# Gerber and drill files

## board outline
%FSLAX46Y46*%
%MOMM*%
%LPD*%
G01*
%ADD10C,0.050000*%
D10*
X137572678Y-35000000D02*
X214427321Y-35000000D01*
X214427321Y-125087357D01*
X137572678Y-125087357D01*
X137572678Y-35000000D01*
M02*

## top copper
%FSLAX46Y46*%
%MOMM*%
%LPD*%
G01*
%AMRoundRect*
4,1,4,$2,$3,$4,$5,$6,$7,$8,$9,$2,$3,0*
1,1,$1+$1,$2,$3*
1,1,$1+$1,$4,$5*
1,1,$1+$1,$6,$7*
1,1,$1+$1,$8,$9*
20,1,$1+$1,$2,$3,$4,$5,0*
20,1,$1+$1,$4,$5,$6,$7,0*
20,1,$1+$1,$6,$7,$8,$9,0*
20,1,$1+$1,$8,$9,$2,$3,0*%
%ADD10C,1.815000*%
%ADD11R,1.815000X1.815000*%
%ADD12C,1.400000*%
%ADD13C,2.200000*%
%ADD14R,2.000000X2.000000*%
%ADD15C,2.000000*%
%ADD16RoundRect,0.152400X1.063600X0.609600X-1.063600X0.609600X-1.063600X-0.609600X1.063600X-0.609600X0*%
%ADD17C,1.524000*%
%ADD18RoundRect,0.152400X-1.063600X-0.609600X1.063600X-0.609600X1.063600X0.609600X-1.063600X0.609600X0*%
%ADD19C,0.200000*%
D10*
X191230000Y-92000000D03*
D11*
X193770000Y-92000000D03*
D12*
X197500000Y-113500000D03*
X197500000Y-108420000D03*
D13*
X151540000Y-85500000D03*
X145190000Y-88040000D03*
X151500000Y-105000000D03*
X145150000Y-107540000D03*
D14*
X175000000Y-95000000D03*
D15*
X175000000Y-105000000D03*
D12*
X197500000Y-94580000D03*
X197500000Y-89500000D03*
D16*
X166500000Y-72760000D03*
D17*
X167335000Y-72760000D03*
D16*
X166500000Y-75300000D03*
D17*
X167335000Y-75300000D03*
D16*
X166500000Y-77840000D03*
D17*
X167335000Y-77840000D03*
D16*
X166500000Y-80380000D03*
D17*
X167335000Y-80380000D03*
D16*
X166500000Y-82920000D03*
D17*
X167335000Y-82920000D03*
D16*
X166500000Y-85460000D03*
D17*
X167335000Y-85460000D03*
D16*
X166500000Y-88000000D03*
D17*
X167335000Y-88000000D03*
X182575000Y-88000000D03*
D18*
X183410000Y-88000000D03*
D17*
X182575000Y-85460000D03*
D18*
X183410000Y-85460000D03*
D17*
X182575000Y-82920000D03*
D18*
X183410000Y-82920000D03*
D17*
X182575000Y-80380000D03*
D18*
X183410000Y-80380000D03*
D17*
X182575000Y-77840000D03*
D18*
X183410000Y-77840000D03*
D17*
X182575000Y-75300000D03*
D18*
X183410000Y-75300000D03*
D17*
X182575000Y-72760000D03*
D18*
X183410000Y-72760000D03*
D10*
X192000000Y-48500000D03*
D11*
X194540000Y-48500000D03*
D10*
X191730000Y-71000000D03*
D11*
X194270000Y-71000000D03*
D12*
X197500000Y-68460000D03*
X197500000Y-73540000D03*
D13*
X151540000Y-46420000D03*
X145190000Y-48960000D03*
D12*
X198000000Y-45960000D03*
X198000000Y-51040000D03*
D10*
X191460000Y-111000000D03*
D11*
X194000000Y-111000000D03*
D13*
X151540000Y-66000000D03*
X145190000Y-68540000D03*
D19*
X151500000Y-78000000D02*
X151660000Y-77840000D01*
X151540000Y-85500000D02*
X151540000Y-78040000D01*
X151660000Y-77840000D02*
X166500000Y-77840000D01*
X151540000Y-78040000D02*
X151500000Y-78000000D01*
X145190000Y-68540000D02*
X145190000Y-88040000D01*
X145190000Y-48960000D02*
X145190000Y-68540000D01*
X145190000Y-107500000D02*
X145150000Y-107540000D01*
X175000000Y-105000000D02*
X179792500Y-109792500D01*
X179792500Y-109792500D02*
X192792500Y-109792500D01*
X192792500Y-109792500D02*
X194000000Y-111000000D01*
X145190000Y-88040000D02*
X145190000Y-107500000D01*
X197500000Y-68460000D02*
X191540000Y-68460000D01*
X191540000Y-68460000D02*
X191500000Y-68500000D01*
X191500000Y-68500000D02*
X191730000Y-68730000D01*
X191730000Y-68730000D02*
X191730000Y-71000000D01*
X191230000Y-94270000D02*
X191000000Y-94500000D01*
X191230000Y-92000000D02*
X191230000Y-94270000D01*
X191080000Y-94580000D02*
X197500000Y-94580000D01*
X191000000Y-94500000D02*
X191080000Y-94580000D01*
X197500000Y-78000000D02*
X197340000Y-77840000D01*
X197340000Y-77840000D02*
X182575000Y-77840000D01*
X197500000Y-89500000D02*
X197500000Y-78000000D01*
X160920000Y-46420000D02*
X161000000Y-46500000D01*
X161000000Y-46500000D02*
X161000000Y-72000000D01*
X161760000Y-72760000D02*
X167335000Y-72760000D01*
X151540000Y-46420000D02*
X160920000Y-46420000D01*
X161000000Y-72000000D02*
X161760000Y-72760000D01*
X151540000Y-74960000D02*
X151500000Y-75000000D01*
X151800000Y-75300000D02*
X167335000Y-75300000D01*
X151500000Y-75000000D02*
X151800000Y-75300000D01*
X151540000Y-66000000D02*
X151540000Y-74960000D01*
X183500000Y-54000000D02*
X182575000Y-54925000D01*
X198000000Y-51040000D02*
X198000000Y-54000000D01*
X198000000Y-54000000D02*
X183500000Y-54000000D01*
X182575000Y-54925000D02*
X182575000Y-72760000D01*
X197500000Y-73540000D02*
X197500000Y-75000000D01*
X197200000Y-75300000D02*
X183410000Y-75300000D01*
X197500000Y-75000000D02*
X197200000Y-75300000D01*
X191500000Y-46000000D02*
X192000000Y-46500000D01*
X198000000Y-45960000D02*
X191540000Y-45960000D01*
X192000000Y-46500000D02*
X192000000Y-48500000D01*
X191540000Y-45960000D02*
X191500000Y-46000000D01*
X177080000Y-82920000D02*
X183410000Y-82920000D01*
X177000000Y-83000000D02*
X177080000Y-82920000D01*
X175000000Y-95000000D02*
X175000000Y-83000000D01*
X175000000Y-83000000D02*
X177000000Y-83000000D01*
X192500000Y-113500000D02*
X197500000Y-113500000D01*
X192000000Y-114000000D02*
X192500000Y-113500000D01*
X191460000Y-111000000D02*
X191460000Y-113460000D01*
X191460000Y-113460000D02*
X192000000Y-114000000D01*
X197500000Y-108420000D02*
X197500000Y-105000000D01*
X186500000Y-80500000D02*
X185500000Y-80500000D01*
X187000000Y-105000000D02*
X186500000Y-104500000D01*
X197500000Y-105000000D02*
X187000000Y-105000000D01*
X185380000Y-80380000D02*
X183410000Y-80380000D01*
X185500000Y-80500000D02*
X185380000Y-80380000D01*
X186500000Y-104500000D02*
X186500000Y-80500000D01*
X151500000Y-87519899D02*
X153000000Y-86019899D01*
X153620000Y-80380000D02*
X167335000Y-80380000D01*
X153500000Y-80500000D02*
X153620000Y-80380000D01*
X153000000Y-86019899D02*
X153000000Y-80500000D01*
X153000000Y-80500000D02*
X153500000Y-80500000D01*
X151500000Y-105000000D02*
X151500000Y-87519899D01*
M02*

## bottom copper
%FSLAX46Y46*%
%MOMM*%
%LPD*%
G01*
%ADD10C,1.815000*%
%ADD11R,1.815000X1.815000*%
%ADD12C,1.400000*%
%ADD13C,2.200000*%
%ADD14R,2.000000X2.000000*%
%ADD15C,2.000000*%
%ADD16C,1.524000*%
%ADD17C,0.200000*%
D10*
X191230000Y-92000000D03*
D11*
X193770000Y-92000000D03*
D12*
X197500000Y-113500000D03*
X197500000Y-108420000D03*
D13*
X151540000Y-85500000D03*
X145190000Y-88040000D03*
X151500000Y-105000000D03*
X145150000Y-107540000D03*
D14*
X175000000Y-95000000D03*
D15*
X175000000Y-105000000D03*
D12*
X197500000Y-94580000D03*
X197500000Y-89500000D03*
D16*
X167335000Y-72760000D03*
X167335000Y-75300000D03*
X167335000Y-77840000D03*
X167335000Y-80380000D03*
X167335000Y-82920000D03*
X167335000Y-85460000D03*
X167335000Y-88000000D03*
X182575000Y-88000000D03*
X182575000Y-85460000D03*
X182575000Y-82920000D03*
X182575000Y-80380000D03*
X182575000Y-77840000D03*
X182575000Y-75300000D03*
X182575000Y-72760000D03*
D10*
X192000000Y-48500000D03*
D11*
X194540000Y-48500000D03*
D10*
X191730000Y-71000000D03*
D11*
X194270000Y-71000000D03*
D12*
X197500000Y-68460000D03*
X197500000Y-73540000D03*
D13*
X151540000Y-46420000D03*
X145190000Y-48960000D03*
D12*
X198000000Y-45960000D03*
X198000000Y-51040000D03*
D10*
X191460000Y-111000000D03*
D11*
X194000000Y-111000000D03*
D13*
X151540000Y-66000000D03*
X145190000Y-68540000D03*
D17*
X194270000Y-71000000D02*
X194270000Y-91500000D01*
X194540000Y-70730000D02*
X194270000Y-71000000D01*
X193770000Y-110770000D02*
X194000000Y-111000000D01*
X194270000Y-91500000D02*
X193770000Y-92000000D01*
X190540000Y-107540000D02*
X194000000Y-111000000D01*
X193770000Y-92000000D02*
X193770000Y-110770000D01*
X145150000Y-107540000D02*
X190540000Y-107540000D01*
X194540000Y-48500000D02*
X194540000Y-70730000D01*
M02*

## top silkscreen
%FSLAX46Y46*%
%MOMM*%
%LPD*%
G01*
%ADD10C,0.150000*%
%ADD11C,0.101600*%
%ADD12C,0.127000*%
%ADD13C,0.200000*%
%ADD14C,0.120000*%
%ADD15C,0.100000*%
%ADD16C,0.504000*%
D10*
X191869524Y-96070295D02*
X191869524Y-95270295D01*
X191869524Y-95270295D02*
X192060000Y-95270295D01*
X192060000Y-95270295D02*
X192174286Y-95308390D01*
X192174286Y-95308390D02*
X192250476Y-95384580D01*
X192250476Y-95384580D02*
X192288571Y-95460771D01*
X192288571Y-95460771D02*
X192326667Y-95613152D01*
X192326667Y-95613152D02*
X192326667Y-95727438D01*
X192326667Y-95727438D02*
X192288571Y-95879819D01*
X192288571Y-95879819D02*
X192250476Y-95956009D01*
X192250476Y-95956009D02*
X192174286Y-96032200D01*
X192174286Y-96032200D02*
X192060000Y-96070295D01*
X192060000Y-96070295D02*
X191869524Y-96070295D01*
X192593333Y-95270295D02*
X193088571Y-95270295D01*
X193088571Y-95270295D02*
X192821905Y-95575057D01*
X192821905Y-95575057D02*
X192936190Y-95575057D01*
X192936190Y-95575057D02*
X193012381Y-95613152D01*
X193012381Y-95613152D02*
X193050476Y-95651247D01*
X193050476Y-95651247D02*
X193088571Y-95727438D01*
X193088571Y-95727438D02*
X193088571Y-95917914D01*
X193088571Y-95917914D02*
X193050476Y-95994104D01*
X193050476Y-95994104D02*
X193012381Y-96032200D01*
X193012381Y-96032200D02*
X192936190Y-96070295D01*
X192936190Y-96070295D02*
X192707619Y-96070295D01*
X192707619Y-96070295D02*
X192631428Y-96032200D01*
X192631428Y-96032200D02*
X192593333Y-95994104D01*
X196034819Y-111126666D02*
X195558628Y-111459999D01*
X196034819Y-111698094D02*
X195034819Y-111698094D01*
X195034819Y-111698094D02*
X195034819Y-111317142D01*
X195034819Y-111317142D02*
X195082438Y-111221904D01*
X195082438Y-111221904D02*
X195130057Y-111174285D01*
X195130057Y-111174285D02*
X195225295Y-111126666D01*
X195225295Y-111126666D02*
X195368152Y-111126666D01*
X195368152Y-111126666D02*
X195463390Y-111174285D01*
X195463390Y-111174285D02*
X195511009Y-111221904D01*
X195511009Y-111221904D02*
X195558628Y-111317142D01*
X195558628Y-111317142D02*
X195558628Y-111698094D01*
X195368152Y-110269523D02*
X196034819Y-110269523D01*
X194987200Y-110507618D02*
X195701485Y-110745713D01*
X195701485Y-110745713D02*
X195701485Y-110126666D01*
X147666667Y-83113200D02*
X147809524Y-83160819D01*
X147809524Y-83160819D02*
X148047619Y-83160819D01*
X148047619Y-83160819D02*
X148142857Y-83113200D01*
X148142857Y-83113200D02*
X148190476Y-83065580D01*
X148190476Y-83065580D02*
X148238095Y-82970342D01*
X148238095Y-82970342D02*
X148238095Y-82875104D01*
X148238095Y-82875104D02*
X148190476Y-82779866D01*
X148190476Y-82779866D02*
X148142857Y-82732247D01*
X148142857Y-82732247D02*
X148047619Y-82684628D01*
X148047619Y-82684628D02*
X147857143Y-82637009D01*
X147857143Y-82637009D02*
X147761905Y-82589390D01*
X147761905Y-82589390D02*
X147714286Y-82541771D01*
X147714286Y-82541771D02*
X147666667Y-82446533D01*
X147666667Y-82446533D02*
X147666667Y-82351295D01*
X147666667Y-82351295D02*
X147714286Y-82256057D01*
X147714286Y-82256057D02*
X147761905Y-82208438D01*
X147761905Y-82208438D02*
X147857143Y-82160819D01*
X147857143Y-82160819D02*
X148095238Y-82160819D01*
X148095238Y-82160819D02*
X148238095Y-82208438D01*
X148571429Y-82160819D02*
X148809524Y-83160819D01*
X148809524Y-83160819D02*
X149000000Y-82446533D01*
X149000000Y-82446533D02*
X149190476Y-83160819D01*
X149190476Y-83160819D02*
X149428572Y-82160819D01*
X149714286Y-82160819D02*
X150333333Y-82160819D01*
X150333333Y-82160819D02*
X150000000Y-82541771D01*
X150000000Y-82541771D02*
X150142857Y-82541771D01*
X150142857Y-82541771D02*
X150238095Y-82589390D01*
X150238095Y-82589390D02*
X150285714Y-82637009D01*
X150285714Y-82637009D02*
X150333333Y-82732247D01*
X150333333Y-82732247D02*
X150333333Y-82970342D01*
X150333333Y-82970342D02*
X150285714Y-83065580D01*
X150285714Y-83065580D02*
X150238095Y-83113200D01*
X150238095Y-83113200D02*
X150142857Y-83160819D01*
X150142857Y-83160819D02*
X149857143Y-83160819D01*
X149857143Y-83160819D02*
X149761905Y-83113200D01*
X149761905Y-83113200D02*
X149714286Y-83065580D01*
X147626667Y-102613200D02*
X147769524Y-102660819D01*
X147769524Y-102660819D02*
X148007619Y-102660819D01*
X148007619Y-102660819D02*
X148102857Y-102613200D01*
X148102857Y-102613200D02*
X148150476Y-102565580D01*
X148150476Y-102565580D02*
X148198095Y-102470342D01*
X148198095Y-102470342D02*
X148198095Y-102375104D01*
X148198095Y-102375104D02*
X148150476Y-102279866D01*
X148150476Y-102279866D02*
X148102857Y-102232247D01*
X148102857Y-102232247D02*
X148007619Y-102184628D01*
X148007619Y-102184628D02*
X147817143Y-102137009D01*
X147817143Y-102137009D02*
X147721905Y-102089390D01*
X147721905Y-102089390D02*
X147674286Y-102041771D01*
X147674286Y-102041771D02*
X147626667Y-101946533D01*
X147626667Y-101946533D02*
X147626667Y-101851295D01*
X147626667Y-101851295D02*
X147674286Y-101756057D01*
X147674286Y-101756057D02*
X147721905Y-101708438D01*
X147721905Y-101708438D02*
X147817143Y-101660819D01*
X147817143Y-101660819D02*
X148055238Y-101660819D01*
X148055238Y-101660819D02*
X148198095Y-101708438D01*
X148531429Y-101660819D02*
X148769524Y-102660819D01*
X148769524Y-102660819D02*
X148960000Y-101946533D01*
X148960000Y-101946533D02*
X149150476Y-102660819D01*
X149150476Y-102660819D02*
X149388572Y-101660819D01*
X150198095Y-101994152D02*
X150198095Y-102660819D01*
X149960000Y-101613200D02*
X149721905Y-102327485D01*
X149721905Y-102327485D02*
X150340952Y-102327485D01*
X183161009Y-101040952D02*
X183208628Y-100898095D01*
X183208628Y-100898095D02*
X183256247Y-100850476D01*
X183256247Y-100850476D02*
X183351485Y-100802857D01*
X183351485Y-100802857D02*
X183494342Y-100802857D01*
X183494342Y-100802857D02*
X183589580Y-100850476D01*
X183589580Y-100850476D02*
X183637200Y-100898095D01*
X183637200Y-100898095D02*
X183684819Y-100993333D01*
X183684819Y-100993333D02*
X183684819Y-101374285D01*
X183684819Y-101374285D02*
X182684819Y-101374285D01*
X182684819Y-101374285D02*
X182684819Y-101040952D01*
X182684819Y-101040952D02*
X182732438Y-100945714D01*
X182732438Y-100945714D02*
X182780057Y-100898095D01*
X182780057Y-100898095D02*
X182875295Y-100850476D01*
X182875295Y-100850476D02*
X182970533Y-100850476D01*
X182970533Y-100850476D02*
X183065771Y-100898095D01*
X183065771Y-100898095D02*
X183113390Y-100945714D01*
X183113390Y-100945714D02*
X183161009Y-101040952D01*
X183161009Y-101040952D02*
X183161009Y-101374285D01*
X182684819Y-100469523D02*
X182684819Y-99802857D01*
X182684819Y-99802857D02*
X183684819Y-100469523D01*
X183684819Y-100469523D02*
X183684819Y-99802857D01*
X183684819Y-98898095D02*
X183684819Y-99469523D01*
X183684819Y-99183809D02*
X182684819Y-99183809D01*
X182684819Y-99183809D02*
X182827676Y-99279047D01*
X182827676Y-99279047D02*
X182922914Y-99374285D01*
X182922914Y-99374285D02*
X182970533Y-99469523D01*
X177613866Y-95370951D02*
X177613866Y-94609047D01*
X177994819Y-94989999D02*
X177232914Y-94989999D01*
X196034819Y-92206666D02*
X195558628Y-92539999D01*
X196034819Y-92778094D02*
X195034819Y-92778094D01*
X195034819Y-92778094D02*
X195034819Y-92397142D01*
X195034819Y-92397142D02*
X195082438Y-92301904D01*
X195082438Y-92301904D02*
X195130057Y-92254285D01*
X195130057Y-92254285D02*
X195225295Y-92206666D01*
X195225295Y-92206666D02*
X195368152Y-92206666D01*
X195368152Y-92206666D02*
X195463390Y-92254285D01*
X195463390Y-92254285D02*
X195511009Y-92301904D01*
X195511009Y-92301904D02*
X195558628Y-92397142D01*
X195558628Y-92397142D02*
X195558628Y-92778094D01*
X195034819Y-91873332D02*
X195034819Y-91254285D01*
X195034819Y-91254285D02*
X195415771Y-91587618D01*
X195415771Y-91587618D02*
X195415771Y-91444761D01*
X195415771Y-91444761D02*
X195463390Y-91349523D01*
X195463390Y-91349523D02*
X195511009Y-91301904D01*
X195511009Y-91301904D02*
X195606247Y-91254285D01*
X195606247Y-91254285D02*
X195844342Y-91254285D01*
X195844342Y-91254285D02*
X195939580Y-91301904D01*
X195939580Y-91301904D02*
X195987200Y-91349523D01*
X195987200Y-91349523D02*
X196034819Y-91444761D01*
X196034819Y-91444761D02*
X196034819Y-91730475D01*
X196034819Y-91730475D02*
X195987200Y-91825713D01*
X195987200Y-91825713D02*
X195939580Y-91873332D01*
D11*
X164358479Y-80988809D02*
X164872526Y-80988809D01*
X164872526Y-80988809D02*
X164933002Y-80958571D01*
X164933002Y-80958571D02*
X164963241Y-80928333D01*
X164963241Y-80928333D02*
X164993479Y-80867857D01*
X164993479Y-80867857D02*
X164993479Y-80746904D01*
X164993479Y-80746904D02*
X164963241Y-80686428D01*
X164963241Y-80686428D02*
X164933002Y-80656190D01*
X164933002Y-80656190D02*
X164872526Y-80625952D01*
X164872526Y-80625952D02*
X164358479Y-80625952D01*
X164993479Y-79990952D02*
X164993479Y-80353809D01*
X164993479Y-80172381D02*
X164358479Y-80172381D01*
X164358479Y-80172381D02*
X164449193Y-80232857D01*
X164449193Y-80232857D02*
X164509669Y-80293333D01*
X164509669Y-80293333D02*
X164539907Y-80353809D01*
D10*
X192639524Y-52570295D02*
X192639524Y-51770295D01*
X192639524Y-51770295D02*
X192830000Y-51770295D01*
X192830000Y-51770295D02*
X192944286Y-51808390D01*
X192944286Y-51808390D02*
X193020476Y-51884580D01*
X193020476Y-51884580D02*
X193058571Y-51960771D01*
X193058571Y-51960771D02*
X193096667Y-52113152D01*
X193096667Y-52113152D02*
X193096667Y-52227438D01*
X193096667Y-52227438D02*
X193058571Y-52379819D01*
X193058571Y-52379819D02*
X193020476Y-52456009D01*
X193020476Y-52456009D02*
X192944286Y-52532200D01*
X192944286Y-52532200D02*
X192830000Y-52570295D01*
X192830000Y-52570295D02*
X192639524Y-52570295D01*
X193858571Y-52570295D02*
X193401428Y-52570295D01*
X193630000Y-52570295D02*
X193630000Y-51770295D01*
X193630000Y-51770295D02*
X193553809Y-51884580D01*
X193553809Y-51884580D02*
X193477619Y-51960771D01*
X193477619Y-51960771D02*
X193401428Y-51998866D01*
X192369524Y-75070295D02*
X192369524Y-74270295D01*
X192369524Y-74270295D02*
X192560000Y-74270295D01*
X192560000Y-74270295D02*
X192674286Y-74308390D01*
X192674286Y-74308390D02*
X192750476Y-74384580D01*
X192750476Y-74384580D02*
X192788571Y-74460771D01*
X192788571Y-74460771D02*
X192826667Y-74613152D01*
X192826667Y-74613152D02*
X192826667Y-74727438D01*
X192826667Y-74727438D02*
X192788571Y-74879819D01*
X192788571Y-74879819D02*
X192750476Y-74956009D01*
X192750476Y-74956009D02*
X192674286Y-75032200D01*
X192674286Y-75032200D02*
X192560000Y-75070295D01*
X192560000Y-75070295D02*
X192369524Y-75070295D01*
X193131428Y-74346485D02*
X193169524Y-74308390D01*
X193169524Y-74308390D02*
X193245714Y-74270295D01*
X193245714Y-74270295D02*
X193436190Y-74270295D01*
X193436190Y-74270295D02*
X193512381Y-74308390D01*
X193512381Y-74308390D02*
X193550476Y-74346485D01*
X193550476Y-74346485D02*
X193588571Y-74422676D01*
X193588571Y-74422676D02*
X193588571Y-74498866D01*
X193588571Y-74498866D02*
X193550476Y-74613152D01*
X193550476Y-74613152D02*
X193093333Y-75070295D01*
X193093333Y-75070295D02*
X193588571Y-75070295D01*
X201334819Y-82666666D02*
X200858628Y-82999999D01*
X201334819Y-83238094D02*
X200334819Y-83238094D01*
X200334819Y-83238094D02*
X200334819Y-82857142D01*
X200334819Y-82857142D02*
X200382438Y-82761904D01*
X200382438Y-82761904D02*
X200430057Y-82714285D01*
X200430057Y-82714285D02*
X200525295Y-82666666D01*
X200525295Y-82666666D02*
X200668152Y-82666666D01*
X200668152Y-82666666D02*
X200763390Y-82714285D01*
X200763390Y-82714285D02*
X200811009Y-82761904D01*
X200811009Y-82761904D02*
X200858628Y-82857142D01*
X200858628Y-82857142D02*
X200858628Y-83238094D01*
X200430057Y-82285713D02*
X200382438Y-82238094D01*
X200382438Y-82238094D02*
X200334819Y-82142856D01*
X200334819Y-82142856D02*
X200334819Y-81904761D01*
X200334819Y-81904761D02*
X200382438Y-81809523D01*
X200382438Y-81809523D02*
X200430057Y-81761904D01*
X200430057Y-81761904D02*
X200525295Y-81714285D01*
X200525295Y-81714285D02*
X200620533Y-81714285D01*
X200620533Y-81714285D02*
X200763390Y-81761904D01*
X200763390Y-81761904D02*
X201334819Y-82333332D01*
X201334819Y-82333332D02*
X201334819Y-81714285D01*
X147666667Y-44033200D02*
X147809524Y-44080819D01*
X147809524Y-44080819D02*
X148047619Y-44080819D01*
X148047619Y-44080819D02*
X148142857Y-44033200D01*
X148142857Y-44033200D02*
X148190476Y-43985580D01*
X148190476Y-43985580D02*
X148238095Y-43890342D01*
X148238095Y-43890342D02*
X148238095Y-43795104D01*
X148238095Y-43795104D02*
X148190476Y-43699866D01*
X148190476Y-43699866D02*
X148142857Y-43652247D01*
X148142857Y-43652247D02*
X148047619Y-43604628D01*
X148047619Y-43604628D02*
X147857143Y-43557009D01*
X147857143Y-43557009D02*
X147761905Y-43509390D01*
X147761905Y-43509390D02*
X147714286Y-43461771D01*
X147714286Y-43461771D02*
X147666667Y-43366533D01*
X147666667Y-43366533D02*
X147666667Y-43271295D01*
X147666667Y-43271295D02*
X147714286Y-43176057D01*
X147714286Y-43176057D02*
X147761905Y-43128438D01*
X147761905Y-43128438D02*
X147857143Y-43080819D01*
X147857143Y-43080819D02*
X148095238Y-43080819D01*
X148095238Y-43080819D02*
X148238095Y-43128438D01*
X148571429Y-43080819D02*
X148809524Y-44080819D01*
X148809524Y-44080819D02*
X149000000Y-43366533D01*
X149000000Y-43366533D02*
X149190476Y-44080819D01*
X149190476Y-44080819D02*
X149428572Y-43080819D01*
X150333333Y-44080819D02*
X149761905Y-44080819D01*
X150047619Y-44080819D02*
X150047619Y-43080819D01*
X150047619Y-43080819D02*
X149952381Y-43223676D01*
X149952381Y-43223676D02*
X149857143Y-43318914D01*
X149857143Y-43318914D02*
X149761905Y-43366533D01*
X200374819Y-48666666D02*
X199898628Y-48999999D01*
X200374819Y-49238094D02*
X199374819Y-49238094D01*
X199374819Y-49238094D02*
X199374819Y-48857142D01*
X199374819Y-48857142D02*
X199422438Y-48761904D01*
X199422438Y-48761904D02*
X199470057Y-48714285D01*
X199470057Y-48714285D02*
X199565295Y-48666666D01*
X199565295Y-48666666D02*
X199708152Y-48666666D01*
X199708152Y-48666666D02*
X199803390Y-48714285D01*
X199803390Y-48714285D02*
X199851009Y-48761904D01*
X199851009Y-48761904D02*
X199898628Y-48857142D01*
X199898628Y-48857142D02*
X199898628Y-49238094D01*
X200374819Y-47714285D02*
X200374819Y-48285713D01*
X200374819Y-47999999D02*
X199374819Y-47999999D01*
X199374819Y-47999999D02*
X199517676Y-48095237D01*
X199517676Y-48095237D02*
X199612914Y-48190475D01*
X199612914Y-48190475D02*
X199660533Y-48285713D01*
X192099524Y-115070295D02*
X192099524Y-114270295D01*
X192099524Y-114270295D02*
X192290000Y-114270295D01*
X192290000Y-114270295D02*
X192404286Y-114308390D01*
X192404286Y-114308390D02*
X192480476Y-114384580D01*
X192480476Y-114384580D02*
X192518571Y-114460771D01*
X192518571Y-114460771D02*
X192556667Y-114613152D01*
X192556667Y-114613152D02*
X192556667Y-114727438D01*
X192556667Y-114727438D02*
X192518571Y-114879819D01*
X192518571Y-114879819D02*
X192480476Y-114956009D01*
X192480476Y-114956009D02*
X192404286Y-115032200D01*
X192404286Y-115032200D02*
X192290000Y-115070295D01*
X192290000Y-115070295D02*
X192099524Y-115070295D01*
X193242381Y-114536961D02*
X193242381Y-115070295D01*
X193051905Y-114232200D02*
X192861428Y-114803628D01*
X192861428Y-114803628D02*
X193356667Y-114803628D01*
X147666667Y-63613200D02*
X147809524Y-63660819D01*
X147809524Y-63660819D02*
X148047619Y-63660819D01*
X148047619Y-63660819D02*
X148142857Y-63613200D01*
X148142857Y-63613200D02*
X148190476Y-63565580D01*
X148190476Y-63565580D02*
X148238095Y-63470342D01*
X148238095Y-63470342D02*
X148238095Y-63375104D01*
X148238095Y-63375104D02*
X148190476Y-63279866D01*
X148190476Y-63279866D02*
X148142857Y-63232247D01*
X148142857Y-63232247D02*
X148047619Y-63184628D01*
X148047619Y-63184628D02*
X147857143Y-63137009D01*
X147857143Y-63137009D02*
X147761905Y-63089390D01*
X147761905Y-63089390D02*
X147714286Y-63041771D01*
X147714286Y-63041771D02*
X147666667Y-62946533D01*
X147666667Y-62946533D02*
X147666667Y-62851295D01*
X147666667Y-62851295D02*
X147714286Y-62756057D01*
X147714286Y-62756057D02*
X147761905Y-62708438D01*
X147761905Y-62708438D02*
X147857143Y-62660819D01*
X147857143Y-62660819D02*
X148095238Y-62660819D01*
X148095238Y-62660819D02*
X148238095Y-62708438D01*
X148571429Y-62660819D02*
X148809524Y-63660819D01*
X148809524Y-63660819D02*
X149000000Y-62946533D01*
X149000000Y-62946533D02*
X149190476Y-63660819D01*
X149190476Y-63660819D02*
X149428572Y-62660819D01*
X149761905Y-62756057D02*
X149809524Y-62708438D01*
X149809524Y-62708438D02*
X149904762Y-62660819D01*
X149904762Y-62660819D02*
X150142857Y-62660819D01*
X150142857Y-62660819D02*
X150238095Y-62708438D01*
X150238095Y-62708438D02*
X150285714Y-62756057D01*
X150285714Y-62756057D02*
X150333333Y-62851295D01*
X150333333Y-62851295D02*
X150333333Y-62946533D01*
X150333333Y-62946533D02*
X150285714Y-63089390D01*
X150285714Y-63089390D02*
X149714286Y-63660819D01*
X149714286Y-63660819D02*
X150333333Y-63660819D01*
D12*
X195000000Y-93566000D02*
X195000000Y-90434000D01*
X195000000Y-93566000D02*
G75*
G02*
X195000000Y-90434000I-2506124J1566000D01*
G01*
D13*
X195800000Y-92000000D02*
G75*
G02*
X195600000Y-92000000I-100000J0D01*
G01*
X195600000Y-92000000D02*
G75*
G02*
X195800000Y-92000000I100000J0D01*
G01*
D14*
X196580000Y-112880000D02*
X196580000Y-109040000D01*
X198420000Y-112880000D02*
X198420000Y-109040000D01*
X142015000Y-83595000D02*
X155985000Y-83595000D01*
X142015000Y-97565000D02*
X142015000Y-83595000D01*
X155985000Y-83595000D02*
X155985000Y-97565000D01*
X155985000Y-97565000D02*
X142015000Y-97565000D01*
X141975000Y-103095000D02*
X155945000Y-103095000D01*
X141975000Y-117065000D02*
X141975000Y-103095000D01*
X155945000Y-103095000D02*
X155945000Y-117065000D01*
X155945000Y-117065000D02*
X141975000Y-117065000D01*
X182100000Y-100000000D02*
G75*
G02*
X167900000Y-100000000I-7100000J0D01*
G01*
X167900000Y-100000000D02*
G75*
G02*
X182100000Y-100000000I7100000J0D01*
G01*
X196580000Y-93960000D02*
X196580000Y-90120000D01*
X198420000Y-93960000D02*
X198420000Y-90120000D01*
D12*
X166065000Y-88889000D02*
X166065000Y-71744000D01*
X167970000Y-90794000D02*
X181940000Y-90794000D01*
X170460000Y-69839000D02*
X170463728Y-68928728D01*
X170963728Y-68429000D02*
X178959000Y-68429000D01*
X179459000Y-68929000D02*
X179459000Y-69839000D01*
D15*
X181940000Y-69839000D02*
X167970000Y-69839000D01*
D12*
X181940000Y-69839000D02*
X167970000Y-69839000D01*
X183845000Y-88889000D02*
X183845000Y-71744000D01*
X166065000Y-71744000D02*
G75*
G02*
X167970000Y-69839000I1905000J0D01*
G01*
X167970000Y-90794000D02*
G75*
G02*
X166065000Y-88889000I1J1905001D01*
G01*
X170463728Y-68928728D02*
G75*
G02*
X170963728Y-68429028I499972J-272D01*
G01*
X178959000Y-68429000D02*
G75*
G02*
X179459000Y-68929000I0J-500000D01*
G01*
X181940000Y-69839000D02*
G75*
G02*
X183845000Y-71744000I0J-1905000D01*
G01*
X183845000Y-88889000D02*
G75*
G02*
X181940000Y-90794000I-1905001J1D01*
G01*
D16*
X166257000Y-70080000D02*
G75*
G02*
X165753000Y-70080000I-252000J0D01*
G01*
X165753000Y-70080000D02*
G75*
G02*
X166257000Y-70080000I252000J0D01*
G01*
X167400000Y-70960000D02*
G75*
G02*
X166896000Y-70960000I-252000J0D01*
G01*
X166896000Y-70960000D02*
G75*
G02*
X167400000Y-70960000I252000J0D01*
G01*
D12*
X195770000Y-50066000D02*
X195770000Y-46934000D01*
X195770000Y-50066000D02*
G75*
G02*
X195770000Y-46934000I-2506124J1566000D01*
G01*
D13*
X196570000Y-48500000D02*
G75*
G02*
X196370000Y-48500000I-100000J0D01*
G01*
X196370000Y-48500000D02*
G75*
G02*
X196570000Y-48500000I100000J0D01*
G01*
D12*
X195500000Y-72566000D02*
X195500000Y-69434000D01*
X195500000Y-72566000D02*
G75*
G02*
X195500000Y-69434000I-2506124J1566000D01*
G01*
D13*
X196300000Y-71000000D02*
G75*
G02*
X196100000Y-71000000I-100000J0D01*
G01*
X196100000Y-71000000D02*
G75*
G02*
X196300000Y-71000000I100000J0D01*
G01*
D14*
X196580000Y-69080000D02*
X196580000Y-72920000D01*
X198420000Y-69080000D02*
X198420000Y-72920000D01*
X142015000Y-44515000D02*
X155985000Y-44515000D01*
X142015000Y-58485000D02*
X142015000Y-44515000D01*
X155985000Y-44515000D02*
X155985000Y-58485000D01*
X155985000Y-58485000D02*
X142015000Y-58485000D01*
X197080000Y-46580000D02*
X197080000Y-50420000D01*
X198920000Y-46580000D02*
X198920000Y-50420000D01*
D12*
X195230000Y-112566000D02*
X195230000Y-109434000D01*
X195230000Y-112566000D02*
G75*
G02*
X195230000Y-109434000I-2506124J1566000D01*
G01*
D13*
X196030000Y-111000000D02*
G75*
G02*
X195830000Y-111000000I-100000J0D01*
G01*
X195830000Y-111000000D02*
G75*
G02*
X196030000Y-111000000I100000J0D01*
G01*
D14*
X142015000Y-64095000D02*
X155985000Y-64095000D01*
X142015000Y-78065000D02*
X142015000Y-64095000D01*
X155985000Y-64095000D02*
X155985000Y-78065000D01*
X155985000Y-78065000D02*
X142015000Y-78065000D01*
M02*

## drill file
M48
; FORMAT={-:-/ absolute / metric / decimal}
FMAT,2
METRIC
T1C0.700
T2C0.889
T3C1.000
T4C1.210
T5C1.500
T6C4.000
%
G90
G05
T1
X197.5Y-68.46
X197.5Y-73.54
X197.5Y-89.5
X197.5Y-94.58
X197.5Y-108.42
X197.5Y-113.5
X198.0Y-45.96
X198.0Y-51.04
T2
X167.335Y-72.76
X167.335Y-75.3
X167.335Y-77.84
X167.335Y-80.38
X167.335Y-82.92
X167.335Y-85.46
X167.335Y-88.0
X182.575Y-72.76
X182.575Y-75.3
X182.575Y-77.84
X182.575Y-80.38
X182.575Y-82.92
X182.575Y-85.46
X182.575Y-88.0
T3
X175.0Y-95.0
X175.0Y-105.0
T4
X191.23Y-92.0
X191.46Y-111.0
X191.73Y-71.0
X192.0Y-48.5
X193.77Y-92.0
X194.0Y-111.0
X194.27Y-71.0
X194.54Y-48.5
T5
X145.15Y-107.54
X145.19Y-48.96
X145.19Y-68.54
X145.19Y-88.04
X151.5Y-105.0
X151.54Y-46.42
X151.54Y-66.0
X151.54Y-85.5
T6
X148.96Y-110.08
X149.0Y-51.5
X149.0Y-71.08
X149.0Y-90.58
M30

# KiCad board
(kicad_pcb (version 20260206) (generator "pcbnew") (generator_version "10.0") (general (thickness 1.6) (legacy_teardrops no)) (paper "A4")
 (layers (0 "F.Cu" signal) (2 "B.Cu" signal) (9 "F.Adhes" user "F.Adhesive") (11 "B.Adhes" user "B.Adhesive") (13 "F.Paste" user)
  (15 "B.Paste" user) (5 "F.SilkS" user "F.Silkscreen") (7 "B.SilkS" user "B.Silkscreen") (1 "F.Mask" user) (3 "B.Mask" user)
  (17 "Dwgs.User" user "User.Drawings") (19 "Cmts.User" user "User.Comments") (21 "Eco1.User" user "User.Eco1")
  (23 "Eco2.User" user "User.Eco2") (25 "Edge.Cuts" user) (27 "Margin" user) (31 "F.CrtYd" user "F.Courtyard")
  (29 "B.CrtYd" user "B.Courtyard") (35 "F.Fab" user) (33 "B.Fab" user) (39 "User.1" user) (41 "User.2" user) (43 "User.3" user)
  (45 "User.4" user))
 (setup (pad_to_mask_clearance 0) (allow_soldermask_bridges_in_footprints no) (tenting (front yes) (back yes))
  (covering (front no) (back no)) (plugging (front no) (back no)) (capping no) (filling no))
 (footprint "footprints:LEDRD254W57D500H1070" (layer "F.Cu") (at 192.5 92 180)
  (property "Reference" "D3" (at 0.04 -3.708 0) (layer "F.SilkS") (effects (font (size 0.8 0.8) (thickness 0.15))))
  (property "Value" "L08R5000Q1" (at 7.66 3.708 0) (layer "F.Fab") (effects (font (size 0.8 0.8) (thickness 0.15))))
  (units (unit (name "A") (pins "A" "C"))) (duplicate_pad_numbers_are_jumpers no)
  (fp_line (start -2.5 -1.566) (end -2.5 1.566) (stroke (width 0.127) (type solid)) (layer "F.SilkS"))
  (fp_arc (start -2.5 -1.566) (mid 2.961291 0) (end -2.5 1.566) (stroke (width 0.127) (type solid)) (layer "F.SilkS"))
  (fp_circle (center -3.2 0) (end -3.1 0) (stroke (width 0.2) (type solid)) (fill no) (layer "F.SilkS"))
  (pad "A" thru_hole circle (at 1.27 0 180) (size 1.815 1.815) (drill 1.21) (layers "*.Cu" "*.Mask") (remove_unused_layers no)
   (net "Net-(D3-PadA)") (solder_mask_margin 0.102))
  (pad "C" thru_hole rect (at -1.27 0 180) (size 1.815 1.815) (drill 1.21) (layers "*.Cu" "*.Mask") (remove_unused_layers no) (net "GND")
   (solder_mask_margin 0.102)))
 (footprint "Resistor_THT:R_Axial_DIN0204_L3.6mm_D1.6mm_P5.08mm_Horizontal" (layer "F.Cu") (at 197.5 113.5 90)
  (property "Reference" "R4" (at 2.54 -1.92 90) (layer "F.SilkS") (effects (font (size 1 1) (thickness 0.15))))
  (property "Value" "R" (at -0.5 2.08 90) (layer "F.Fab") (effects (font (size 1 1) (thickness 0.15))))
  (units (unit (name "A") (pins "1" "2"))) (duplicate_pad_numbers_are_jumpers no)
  (fp_line (start 0.62 -0.92) (end 4.46 -0.92) (stroke (width 0.12) (type solid)) (layer "F.SilkS"))
  (fp_line (start 0.62 0.92) (end 4.46 0.92) (stroke (width 0.12) (type solid)) (layer "F.SilkS"))
  (pad "1" thru_hole circle (at 0 0 90) (size 1.4 1.4) (drill 0.7) (layers "*.Cu" "*.Mask") (remove_unused_layers no) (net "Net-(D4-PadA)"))
  (pad "2" thru_hole circle (at 5.08 0 90) (size 1.4 1.4) (drill 0.7) (layers "*.Cu" "*.Mask") (remove_unused_layers no) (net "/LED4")))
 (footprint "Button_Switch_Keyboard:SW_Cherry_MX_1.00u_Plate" (layer "F.Cu") (at 151.54 85.5)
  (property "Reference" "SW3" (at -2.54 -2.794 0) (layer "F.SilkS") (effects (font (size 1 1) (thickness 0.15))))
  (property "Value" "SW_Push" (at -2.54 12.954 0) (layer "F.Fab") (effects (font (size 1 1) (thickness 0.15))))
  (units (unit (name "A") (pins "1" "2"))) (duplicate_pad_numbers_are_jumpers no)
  (fp_line (start -9.525 -1.905) (end 4.445 -1.905) (stroke (width 0.12) (type solid)) (layer "F.SilkS"))
  (fp_line (start -9.525 12.065) (end -9.525 -1.905) (stroke (width 0.12) (type solid)) (layer "F.SilkS"))
  (fp_line (start 4.445 -1.905) (end 4.445 12.065) (stroke (width 0.12) (type solid)) (layer "F.SilkS"))
  (fp_line (start 4.445 12.065) (end -9.525 12.065) (stroke (width 0.12) (type solid)) (layer "F.SilkS"))
  (pad "" np_thru_hole circle (at -2.54 5.08) (size 4 4) (drill 4) (layers "*.Cu" "*.Mask"))
  (pad "1" thru_hole circle (at 0 0) (size 2.2 2.2) (drill 1.5) (layers "*.Cu" "*.Mask") (remove_unused_layers no) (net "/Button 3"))
  (pad "2" thru_hole circle (at -6.35 2.54) (size 2.2 2.2) (drill 1.5) (layers "*.Cu" "*.Mask") (remove_unused_layers no) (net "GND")))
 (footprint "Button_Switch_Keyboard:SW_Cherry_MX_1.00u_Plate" (layer "F.Cu") (at 151.5 105)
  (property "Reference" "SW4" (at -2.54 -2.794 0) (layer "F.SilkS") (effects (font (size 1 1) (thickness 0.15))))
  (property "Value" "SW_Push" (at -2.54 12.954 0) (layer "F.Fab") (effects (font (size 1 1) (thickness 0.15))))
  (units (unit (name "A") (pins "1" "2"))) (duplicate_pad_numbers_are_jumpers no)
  (fp_line (start -9.525 -1.905) (end 4.445 -1.905) (stroke (width 0.12) (type solid)) (layer "F.SilkS"))
  (fp_line (start -9.525 12.065) (end -9.525 -1.905) (stroke (width 0.12) (type solid)) (layer "F.SilkS"))
  (fp_line (start 4.445 -1.905) (end 4.445 12.065) (stroke (width 0.12) (type solid)) (layer "F.SilkS"))
  (fp_line (start 4.445 12.065) (end -9.525 12.065) (stroke (width 0.12) (type solid)) (layer "F.SilkS"))
  (pad "" np_thru_hole circle (at -2.54 5.08) (size 4 4) (drill 4) (layers "*.Cu" "*.Mask"))
  (pad "1" thru_hole circle (at 0 0) (size 2.2 2.2) (drill 1.5) (layers "*.Cu" "*.Mask") (remove_unused_layers no) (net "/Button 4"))
  (pad "2" thru_hole circle (at -6.35 2.54) (size 2.2 2.2) (drill 1.5) (layers "*.Cu" "*.Mask") (remove_unused_layers no) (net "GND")))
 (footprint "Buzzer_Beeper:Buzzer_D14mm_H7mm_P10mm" (layer "F.Cu") (at 175 95 -90)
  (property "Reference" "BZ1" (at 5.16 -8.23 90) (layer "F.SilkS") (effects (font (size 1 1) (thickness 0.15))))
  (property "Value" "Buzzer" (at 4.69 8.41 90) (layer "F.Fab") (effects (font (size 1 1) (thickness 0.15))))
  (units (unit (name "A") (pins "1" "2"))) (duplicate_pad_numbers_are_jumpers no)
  (fp_circle (center 5 0) (end 12.1 0) (stroke (width 0.12) (type solid)) (fill no) (layer "F.SilkS"))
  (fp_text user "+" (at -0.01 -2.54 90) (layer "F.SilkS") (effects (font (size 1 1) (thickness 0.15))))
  (pad "1" thru_hole rect (at 0 0 270) (size 2 2) (drill 1) (layers "*.Cu" "*.Mask") (remove_unused_layers no) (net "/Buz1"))
  (pad "2" thru_hole circle (at 10 0 270) (size 2 2) (drill 1) (layers "*.Cu" "*.Mask") (remove_unused_layers no) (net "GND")))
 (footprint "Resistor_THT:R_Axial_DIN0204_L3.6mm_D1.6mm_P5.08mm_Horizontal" (layer "F.Cu") (at 197.5 94.58 90)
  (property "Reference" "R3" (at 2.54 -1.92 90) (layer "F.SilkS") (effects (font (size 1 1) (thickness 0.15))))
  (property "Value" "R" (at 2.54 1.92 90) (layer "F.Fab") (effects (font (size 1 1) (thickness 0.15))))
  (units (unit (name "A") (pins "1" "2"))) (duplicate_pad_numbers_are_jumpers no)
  (fp_line (start 0.62 -0.92) (end 4.46 -0.92) (stroke (width 0.12) (type solid)) (layer "F.SilkS"))
  (fp_line (start 0.62 0.92) (end 4.46 0.92) (stroke (width 0.12) (type solid)) (layer "F.SilkS"))
  (pad "1" thru_hole circle (at 0 0 90) (size 1.4 1.4) (drill 0.7) (layers "*.Cu" "*.Mask") (remove_unused_layers no) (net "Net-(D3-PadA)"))
  (pad "2" thru_hole circle (at 5.08 0 90) (size 1.4 1.4) (drill 0.7) (layers "*.Cu" "*.Mask") (remove_unused_layers no) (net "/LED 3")))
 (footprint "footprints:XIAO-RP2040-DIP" (layer "F.Cu") (at 174.955 80.38 90)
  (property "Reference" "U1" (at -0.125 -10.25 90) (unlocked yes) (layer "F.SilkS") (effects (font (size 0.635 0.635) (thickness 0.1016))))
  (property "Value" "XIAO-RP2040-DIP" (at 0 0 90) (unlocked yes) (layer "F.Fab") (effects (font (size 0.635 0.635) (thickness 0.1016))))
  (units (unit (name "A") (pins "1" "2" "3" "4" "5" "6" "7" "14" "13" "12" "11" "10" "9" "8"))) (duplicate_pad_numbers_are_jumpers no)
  (fp_line (start -8.509 -8.89) (end 8.636 -8.89) (stroke (width 0.127) (type solid)) (layer "F.SilkS"))
  (fp_line (start -10.414 -6.985) (end -10.414 6.985) (stroke (width 0.127) (type solid)) (layer "F.SilkS"))
  (fp_line (start 10.541 -4.495) (end 11.451272 -4.491272) (stroke (width 0.127) (type solid)) (layer "F.SilkS"))
  (fp_line (start 11.951 -3.991272) (end 11.951 4.004) (stroke (width 0.127) (type solid)) (layer "F.SilkS"))
  (fp_line (start 11.451 4.504) (end 10.541 4.504) (stroke (width 0.127) (type solid)) (layer "F.SilkS"))
  (fp_line (start 10.541 6.985) (end 10.541 -6.985) (stroke (width 0.1) (type solid)) (layer "F.SilkS"))
  (fp_line (start 10.541 6.985) (end 10.541 -6.985) (stroke (width 0.127) (type solid)) (layer "F.SilkS"))
  (fp_line (start -8.509 8.89) (end 8.636 8.89) (stroke (width 0.127) (type solid)) (layer "F.SilkS"))
  (fp_arc (start 8.636 -8.89) (mid 9.983038 -8.332038) (end 10.541 -6.985) (stroke (width 0.127) (type solid)) (layer "F.SilkS"))
  (fp_arc (start -10.414 -6.985) (mid -9.856038 -8.332038) (end -8.509 -8.89) (stroke (width 0.127) (type solid)) (layer "F.SilkS"))
  (fp_arc (start 11.451272 -4.491272) (mid 11.804644 -4.344724) (end 11.951 -3.991272) (stroke (width 0.127) (type default))
   (layer "F.SilkS"))
  (fp_arc (start 11.951 4.004) (mid 11.804553 4.357553) (end 11.451 4.504) (stroke (width 0.127) (type default)) (layer "F.SilkS"))
  (fp_arc (start 10.541 6.985) (mid 9.983038 8.332038) (end 8.636 8.89) (stroke (width 0.127) (type solid)) (layer "F.SilkS"))
  (fp_arc (start -8.509 8.89) (mid -9.856038 8.332038) (end -10.414 6.985) (stroke (width 0.127) (type solid)) (layer "F.SilkS"))
  (fp_circle (center 10.3 -8.95) (end 10.554 -8.95) (stroke (width 0.5) (type solid)) (fill yes) (layer "F.SilkS"))
  (fp_circle (center 9.42 -7.807) (end 9.674 -7.807) (stroke (width 0.5) (type solid)) (fill yes) (layer "F.SilkS"))
  (pad "1" smd roundrect (at 7.62 -8.455 180) (size 2.432 1.524) (layers "F.Cu" "F.Mask") (roundrect_rratio 0.1) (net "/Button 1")
   (thermal_bridge_angle 45))
  (pad "1" thru_hole circle (at 7.62 -7.62 180) (size 1.524 1.524) (drill 0.889) (layers "*.Cu" "*.Mask") (remove_unused_layers no)
   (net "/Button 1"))
  (pad "2" smd roundrect (at 5.08 -8.455 180) (size 2.432 1.524) (layers "F.Cu" "F.Mask") (roundrect_rratio 0.1) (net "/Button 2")
   (thermal_bridge_angle 45))
  (pad "2" thru_hole circle (at 5.08 -7.62 180) (size 1.524 1.524) (drill 0.889) (layers "*.Cu" "*.Mask") (remove_unused_layers no)
   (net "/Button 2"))
  (pad "3" smd roundrect (at 2.54 -8.455 180) (size 2.432 1.524) (layers "F.Cu" "F.Mask") (roundrect_rratio 0.1) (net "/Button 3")
   (thermal_bridge_angle 45))
  (pad "3" thru_hole circle (at 2.54 -7.62 180) (size 1.524 1.524) (drill 0.889) (layers "*.Cu" "*.Mask") (remove_unused_layers no)
   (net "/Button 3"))
  (pad "4" smd roundrect (at 0 -8.455 180) (size 2.432 1.524) (layers "F.Cu" "F.Mask") (roundrect_rratio 0.1) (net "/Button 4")
   (thermal_bridge_angle 45))
  (pad "4" thru_hole circle (at 0 -7.62 180) (size 1.524 1.524) (drill 0.889) (layers "*.Cu" "*.Mask") (remove_unused_layers no)
   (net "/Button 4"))
  (pad "5" smd roundrect (at -2.54 -8.455 180) (size 2.432 1.524) (layers "F.Cu" "F.Mask") (roundrect_rratio 0.1)
   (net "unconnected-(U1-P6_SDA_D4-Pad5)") (thermal_bridge_angle 45))
  (pad "5" thru_hole circle (at -2.54 -7.62 180) (size 1.524 1.524) (drill 0.889) (layers "*.Cu" "*.Mask") (remove_unused_layers no)
   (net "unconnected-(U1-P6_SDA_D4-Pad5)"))
  (pad "6" smd roundrect (at -5.08 -8.455 180) (size 2.432 1.524) (layers "F.Cu" "F.Mask") (roundrect_rratio 0.1)
   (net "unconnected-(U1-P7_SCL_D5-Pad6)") (thermal_bridge_angle 45))
  (pad "6" thru_hole circle (at -5.08 -7.62 180) (size 1.524 1.524) (drill 0.889) (layers "*.Cu" "*.Mask") (remove_unused_layers no)
   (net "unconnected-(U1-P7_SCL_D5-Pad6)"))
  (pad "7" smd roundrect (at -7.62 -8.455 180) (size 2.432 1.524) (layers "F.Cu" "F.Mask") (roundrect_rratio 0.1)
   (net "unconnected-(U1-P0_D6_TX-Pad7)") (thermal_bridge_angle 45))
  (pad "7" thru_hole circle (at -7.62 -7.62 180) (size 1.524 1.524) (drill 0.889) (layers "*.Cu" "*.Mask") (remove_unused_layers no)
   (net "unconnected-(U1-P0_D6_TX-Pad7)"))
  (pad "8" thru_hole circle (at -7.62 7.62) (size 1.524 1.524) (drill 0.889) (layers "*.Cu" "*.Mask") (remove_unused_layers no)
   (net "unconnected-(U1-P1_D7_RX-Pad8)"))
  (pad "8" smd roundrect (at -7.62 8.455) (size 2.432 1.524) (layers "F.Cu" "F.Mask") (roundrect_rratio 0.1)
   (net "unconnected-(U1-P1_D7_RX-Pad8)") (thermal_bridge_angle 45))
  (pad "9" thru_hole circle (at -5.08 7.62) (size 1.524 1.524) (drill 0.889) (layers "*.Cu" "*.Mask") (remove_unused_layers no)
   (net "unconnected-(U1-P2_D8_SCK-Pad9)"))
  (pad "9" smd roundrect (at -5.08 8.455) (size 2.432 1.524) (layers "F.Cu" "F.Mask") (roundrect_rratio 0.1)
   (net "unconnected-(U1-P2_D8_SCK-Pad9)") (thermal_bridge_angle 45))
  (pad "10" thru_hole circle (at -2.54 7.62) (size 1.524 1.524) (drill 0.889) (layers "*.Cu" "*.Mask") (remove_unused_layers no)
   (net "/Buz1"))
  (pad "10" smd roundrect (at -2.54 8.455) (size 2.432 1.524) (layers "F.Cu" "F.Mask") (roundrect_rratio 0.1) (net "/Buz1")
   (thermal_bridge_angle 45))
  (pad "11" thru_hole circle (at 0 7.62) (size 1.524 1.524) (drill 0.889) (layers "*.Cu" "*.Mask") (remove_unused_layers no) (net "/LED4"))
  (pad "11" smd roundrect (at 0 8.455) (size 2.432 1.524) (layers "F.Cu" "F.Mask") (roundrect_rratio 0.1) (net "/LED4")
   (thermal_bridge_angle 45))
  (pad "12" thru_hole circle (at 2.54 7.62) (size 1.524 1.524) (drill 0.889) (layers "*.Cu" "*.Mask") (remove_unused_layers no)
   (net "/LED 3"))
  (pad "12" smd roundrect (at 2.54 8.455) (size 2.432 1.524) (layers "F.Cu" "F.Mask") (roundrect_rratio 0.1) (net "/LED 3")
   (thermal_bridge_angle 45))
  (pad "13" thru_hole circle (at 5.08 7.62) (size 1.524 1.524) (drill 0.889) (layers "*.Cu" "*.Mask") (remove_unused_layers no)
   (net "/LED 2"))
  (pad "13" smd roundrect (at 5.08 8.455) (size 2.432 1.524) (layers "F.Cu" "F.Mask") (roundrect_rratio 0.1) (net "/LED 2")
   (thermal_bridge_angle 45))
  (pad "14" thru_hole circle (at 7.62 7.62) (size 1.524 1.524) (drill 0.889) (layers "*.Cu" "*.Mask") (remove_unused_layers no)
   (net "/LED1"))
  (pad "14" smd roundrect (at 7.62 8.455) (size 2.432 1.524) (layers "F.Cu" "F.Mask") (roundrect_rratio 0.1) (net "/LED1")
   (thermal_bridge_angle 45)))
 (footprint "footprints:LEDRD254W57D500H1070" (layer "F.Cu") (at 193.27 48.5 180)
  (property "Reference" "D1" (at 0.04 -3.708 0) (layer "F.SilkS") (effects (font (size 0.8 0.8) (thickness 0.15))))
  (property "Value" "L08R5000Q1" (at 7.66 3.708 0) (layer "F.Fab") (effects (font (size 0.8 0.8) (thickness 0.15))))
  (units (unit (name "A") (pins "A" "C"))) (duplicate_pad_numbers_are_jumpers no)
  (fp_line (start -2.5 -1.566) (end -2.5 1.566) (stroke (width 0.127) (type solid)) (layer "F.SilkS"))
  (fp_arc (start -2.5 -1.566) (mid 2.961291 0) (end -2.5 1.566) (stroke (width 0.127) (type solid)) (layer "F.SilkS"))
  (fp_circle (center -3.2 0) (end -3.1 0) (stroke (width 0.2) (type solid)) (fill no) (layer "F.SilkS"))
  (pad "A" thru_hole circle (at 1.27 0 180) (size 1.815 1.815) (drill 1.21) (layers "*.Cu" "*.Mask") (remove_unused_layers no)
   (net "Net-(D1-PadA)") (solder_mask_margin 0.102))
  (pad "C" thru_hole rect (at -1.27 0 180) (size 1.815 1.815) (drill 1.21) (layers "*.Cu" "*.Mask") (remove_unused_layers no) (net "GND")
   (solder_mask_margin 0.102)))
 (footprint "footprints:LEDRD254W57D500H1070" (layer "F.Cu") (at 193 71 180)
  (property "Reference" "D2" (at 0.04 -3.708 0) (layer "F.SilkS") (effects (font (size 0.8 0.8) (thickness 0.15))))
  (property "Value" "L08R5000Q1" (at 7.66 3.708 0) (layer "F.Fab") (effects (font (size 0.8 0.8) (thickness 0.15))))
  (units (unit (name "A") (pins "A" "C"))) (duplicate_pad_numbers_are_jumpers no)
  (fp_line (start -2.5 -1.566) (end -2.5 1.566) (stroke (width 0.127) (type solid)) (layer "F.SilkS"))
  (fp_arc (start -2.5 -1.566) (mid 2.961291 0) (end -2.5 1.566) (stroke (width 0.127) (type solid)) (layer "F.SilkS"))
  (fp_circle (center -3.2 0) (end -3.1 0) (stroke (width 0.2) (type solid)) (fill no) (layer "F.SilkS"))
  (pad "A" thru_hole circle (at 1.27 0 180) (size 1.815 1.815) (drill 1.21) (layers "*.Cu" "*.Mask") (remove_unused_layers no)
   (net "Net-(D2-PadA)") (solder_mask_margin 0.102))
  (pad "C" thru_hole rect (at -1.27 0 180) (size 1.815 1.815) (drill 1.21) (layers "*.Cu" "*.Mask") (remove_unused_layers no) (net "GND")
   (solder_mask_margin 0.102)))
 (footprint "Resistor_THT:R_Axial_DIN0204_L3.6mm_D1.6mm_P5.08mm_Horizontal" (layer "F.Cu") (at 197.5 68.46 -90)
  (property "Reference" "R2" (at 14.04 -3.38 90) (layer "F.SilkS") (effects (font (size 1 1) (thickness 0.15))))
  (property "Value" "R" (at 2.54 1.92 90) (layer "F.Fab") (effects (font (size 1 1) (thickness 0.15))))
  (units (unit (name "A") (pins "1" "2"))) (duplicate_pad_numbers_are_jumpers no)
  (fp_line (start 0.62 0.92) (end 4.46 0.92) (stroke (width 0.12) (type solid)) (layer "F.SilkS"))
  (fp_line (start 0.62 -0.92) (end 4.46 -0.92) (stroke (width 0.12) (type solid)) (layer "F.SilkS"))
  (pad "1" thru_hole circle (at 0 0 270) (size 1.4 1.4) (drill 0.7) (layers "*.Cu" "*.Mask") (remove_unused_layers no) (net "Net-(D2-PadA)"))
  (pad "2" thru_hole circle (at 5.08 0 270) (size 1.4 1.4) (drill 0.7) (layers "*.Cu" "*.Mask") (remove_unused_layers no) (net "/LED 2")))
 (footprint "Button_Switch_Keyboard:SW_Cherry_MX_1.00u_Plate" (layer "F.Cu") (at 151.54 46.42)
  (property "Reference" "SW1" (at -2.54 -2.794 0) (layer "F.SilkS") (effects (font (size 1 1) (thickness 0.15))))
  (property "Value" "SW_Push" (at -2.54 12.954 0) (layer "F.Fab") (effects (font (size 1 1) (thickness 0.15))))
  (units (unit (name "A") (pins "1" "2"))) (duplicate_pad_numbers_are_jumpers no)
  (fp_line (start -9.525 -1.905) (end 4.445 -1.905) (stroke (width 0.12) (type solid)) (layer "F.SilkS"))
  (fp_line (start -9.525 12.065) (end -9.525 -1.905) (stroke (width 0.12) (type solid)) (layer "F.SilkS"))
  (fp_line (start 4.445 -1.905) (end 4.445 12.065) (stroke (width 0.12) (type solid)) (layer "F.SilkS"))
  (fp_line (start 4.445 12.065) (end -9.525 12.065) (stroke (width 0.12) (type solid)) (layer "F.SilkS"))
  (pad "" np_thru_hole circle (at -2.54 5.08) (size 4 4) (drill 4) (layers "*.Cu" "*.Mask"))
  (pad "1" thru_hole circle (at 0 0) (size 2.2 2.2) (drill 1.5) (layers "*.Cu" "*.Mask") (remove_unused_layers no) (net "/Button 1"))
  (pad "2" thru_hole circle (at -6.35 2.54) (size 2.2 2.2) (drill 1.5) (layers "*.Cu" "*.Mask") (remove_unused_layers no) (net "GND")))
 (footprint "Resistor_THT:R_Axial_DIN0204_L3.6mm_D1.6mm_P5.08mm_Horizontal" (layer "F.Cu") (at 198 45.96 -90)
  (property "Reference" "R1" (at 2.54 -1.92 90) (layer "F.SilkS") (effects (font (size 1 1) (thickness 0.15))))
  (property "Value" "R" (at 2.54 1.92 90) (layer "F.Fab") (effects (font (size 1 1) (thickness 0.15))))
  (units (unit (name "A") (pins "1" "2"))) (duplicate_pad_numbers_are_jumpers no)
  (fp_line (start 0.62 0.92) (end 4.46 0.92) (stroke (width 0.12) (type solid)) (layer "F.SilkS"))
  (fp_line (start 0.62 -0.92) (end 4.46 -0.92) (stroke (width 0.12) (type solid)) (layer "F.SilkS"))
  (pad "1" thru_hole circle (at 0 0 270) (size 1.4 1.4) (drill 0.7) (layers "*.Cu" "*.Mask") (remove_unused_layers no) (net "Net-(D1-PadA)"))
  (pad "2" thru_hole circle (at 5.08 0 270) (size 1.4 1.4) (drill 0.7) (layers "*.Cu" "*.Mask") (remove_unused_layers no) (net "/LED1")))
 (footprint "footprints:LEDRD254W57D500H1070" (layer "F.Cu") (at 192.73 111 180)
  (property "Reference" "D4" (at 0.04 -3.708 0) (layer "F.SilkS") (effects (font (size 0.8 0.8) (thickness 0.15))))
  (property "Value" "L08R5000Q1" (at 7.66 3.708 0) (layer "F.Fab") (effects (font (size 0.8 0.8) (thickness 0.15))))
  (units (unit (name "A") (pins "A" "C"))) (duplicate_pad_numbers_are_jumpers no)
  (fp_line (start -2.5 -1.566) (end -2.5 1.566) (stroke (width 0.127) (type solid)) (layer "F.SilkS"))
  (fp_arc (start -2.5 -1.566) (mid 2.961291 0) (end -2.5 1.566) (stroke (width 0.127) (type solid)) (layer "F.SilkS"))
  (fp_circle (center -3.2 0) (end -3.1 0) (stroke (width 0.2) (type solid)) (fill no) (layer "F.SilkS"))
  (pad "A" thru_hole circle (at 1.27 0 180) (size 1.815 1.815) (drill 1.21) (layers "*.Cu" "*.Mask") (remove_unused_layers no)
   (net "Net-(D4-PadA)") (solder_mask_margin 0.102))
  (pad "C" thru_hole rect (at -1.27 0 180) (size 1.815 1.815) (drill 1.21) (layers "*.Cu" "*.Mask") (remove_unused_layers no) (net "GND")
   (solder_mask_margin 0.102)))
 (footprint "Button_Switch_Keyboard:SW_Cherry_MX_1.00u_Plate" (layer "F.Cu") (at 151.54 66)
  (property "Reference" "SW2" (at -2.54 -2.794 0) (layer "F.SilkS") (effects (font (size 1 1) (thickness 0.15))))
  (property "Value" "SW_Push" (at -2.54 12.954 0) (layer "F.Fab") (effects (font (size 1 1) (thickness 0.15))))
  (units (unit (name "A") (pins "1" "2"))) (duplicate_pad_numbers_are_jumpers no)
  (fp_line (start -9.525 -1.905) (end 4.445 -1.905) (stroke (width 0.12) (type solid)) (layer "F.SilkS"))
  (fp_line (start -9.525 12.065) (end -9.525 -1.905) (stroke (width 0.12) (type solid)) (layer "F.SilkS"))
  (fp_line (start 4.445 -1.905) (end 4.445 12.065) (stroke (width 0.12) (type solid)) (layer "F.SilkS"))
  (fp_line (start 4.445 12.065) (end -9.525 12.065) (stroke (width 0.12) (type solid)) (layer "F.SilkS"))
  (pad "" np_thru_hole circle (at -2.54 5.08) (size 4 4) (drill 4) (layers "*.Cu" "*.Mask"))
  (pad "1" thru_hole circle (at 0 0) (size 2.2 2.2) (drill 1.5) (layers "*.Cu" "*.Mask") (remove_unused_layers no) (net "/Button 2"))
  (pad "2" thru_hole circle (at -6.35 2.54) (size 2.2 2.2) (drill 1.5) (layers "*.Cu" "*.Mask") (remove_unused_layers no) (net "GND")))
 (gr_rect (start 137.572678 35) (end 214.427321 125.087357) (stroke (width 0.05) (type default)) (fill no) (layer "Edge.Cuts"))
 (segment (start 151.5 78) (end 151.66 77.84) (width 0.2) (layer "F.Cu") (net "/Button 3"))
 (segment (start 151.54 85.5) (end 151.54 78.04) (width 0.2) (layer "F.Cu") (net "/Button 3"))
 (segment (start 151.66 77.84) (end 166.5 77.84) (width 0.2) (layer "F.Cu") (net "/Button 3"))
 (segment (start 151.54 78.04) (end 151.5 78) (width 0.2) (layer "F.Cu") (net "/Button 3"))
 (segment (start 145.19 68.54) (end 145.19 88.04) (width 0.2) (layer "F.Cu") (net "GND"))
 (segment (start 145.19 48.96) (end 145.19 68.54) (width 0.2) (layer "F.Cu") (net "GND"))
 (segment (start 145.19 107.5) (end 145.15 107.54) (width 0.2) (layer "F.Cu") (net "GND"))
 (segment (start 175 105) (end 179.7925 109.7925) (width 0.2) (layer "F.Cu") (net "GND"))
 (segment (start 179.7925 109.7925) (end 192.7925 109.7925) (width 0.2) (layer "F.Cu") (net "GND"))
 (segment (start 192.7925 109.7925) (end 194 111) (width 0.2) (layer "F.Cu") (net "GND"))
 (segment (start 145.19 88.04) (end 145.19 107.5) (width 0.2) (layer "F.Cu") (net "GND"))
 (segment (start 194.27 71) (end 194.27 91.5) (width 0.2) (layer "B.Cu") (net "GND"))
 (segment (start 194.54 70.73) (end 194.27 71) (width 0.2) (layer "B.Cu") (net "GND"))
 (segment (start 193.77 110.77) (end 194 111) (width 0.2) (layer "B.Cu") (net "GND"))
 (segment (start 194.27 91.5) (end 193.77 92) (width 0.2) (layer "B.Cu") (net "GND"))
 (segment (start 190.54 107.54) (end 194 111) (width 0.2) (layer "B.Cu") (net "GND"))
 (segment (start 193.77 92) (end 193.77 110.77) (width 0.2) (layer "B.Cu") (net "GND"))
 (segment (start 145.15 107.54) (end 190.54 107.54) (width 0.2) (layer "B.Cu") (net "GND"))
 (segment (start 194.54 48.5) (end 194.54 70.73) (width 0.2) (layer "B.Cu") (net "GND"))
 (segment (start 197.5 68.46) (end 191.54 68.46) (width 0.2) (layer "F.Cu") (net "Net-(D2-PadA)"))
 (segment (start 191.54 68.46) (end 191.5 68.5) (width 0.2) (layer "F.Cu") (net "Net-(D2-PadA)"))
 (segment (start 191.5 68.5) (end 191.73 68.73) (width 0.2) (layer "F.Cu") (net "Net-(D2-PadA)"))
 (segment (start 191.73 68.73) (end 191.73 71) (width 0.2) (layer "F.Cu") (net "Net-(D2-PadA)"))
 (segment (start 191.23 94.27) (end 191 94.5) (width 0.2) (layer "F.Cu") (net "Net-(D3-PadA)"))
 (segment (start 191.23 92) (end 191.23 94.27) (width 0.2) (layer "F.Cu") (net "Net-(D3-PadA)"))
 (segment (start 191.08 94.58) (end 197.5 94.58) (width 0.2) (layer "F.Cu") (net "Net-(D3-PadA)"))
 (segment (start 191 94.5) (end 191.08 94.58) (width 0.2) (layer "F.Cu") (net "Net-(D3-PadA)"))
 (segment (start 197.5 78) (end 197.34 77.84) (width 0.2) (layer "F.Cu") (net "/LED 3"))
 (segment (start 197.34 77.84) (end 182.575 77.84) (width 0.2) (layer "F.Cu") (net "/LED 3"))
 (segment (start 197.5 89.5) (end 197.5 78) (width 0.2) (layer "F.Cu") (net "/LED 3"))
 (segment (start 160.92 46.42) (end 161 46.5) (width 0.2) (layer "F.Cu") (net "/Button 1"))
 (segment (start 161 46.5) (end 161 72) (width 0.2) (layer "F.Cu") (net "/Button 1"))
 (segment (start 161.76 72.76) (end 167.335 72.76) (width 0.2) (layer "F.Cu") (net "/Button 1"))
 (segment (start 151.54 46.42) (end 160.92 46.42) (width 0.2) (layer "F.Cu") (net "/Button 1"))
 (segment (start 161 72) (end 161.76 72.76) (width 0.2) (layer "F.Cu") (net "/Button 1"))
 (segment (start 151.54 74.96) (end 151.5 75) (width 0.2) (layer "F.Cu") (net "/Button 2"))
 (segment (start 151.8 75.3) (end 167.335 75.3) (width 0.2) (layer "F.Cu") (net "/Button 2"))
 (segment (start 151.5 75) (end 151.8 75.3) (width 0.2) (layer "F.Cu") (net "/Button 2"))
 (segment (start 151.54 66) (end 151.54 74.96) (width 0.2) (layer "F.Cu") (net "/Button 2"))
 (segment (start 183.5 54) (end 182.575 54.925) (width 0.2) (layer "F.Cu") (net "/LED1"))
 (segment (start 198 51.04) (end 198 54) (width 0.2) (layer "F.Cu") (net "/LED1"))
 (segment (start 198 54) (end 183.5 54) (width 0.2) (layer "F.Cu") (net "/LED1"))
 (segment (start 182.575 54.925) (end 182.575 72.76) (width 0.2) (layer "F.Cu") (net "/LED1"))
 (segment (start 197.5 73.54) (end 197.5 75) (width 0.2) (layer "F.Cu") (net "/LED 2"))
 (segment (start 197.2 75.3) (end 183.41 75.3) (width 0.2) (layer "F.Cu") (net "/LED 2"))
 (segment (start 197.5 75) (end 197.2 75.3) (width 0.2) (layer "F.Cu") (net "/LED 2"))
 (segment (start 191.5 46) (end 192 46.5) (width 0.2) (layer "F.Cu") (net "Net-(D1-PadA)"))
 (segment (start 198 45.96) (end 191.54 45.96) (width 0.2) (layer "F.Cu") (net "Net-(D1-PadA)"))
 (segment (start 192 46.5) (end 192 48.5) (width 0.2) (layer "F.Cu") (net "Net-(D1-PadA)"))
 (segment (start 191.54 45.96) (end 191.5 46) (width 0.2) (layer "F.Cu") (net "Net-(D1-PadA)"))
 (segment (start 177.08 82.92) (end 183.41 82.92) (width 0.2) (layer "F.Cu") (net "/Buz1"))
 (segment (start 177 83) (end 177.08 82.92) (width 0.2) (layer "F.Cu") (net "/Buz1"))
 (segment (start 175 95) (end 175 83) (width 0.2) (layer "F.Cu") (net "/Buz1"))
 (segment (start 175 83) (end 177 83) (width 0.2) (layer "F.Cu") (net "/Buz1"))
 (segment (start 192.5 113.5) (end 197.5 113.5) (width 0.2) (layer "F.Cu") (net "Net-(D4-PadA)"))
 (segment (start 192 114) (end 192.5 113.5) (width 0.2) (layer "F.Cu") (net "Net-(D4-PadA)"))
 (segment (start 191.46 111) (end 191.46 113.46) (width 0.2) (layer "F.Cu") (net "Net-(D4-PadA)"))
 (segment (start 191.46 113.46) (end 192 114) (width 0.2) (layer "F.Cu") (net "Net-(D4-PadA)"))
 (segment (start 197.5 108.42) (end 197.5 105) (width 0.2) (layer "F.Cu") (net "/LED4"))
 (segment (start 186.5 80.5) (end 185.5 80.5) (width 0.2) (layer "F.Cu") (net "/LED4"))
 (segment (start 187 105) (end 186.5 104.5) (width 0.2) (layer "F.Cu") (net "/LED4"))
 (segment (start 197.5 105) (end 187 105) (width 0.2) (layer "F.Cu") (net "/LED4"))
 (segment (start 185.38 80.38) (end 183.41 80.38) (width 0.2) (layer "F.Cu") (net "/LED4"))
 (segment (start 185.5 80.5) (end 185.38 80.38) (width 0.2) (layer "F.Cu") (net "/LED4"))
 (segment (start 186.5 104.5) (end 186.5 80.5) (width 0.2) (layer "F.Cu") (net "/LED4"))
 (segment (start 151.5 87.519899) (end 153 86.019899) (width 0.2) (layer "F.Cu") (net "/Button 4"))
 (segment (start 153.62 80.38) (end 167.335 80.38) (width 0.2) (layer "F.Cu") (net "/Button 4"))
 (segment (start 153.5 80.5) (end 153.62 80.38) (width 0.2) (layer "F.Cu") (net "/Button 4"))
 (segment (start 153 86.019899) (end 153 80.5) (width 0.2) (layer "F.Cu") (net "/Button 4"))
 (segment (start 153 80.5) (end 153.5 80.5) (width 0.2) (layer "F.Cu") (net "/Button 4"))
 (segment (start 151.5 105) (end 151.5 87.519899) (width 0.2) (layer "F.Cu") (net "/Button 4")))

